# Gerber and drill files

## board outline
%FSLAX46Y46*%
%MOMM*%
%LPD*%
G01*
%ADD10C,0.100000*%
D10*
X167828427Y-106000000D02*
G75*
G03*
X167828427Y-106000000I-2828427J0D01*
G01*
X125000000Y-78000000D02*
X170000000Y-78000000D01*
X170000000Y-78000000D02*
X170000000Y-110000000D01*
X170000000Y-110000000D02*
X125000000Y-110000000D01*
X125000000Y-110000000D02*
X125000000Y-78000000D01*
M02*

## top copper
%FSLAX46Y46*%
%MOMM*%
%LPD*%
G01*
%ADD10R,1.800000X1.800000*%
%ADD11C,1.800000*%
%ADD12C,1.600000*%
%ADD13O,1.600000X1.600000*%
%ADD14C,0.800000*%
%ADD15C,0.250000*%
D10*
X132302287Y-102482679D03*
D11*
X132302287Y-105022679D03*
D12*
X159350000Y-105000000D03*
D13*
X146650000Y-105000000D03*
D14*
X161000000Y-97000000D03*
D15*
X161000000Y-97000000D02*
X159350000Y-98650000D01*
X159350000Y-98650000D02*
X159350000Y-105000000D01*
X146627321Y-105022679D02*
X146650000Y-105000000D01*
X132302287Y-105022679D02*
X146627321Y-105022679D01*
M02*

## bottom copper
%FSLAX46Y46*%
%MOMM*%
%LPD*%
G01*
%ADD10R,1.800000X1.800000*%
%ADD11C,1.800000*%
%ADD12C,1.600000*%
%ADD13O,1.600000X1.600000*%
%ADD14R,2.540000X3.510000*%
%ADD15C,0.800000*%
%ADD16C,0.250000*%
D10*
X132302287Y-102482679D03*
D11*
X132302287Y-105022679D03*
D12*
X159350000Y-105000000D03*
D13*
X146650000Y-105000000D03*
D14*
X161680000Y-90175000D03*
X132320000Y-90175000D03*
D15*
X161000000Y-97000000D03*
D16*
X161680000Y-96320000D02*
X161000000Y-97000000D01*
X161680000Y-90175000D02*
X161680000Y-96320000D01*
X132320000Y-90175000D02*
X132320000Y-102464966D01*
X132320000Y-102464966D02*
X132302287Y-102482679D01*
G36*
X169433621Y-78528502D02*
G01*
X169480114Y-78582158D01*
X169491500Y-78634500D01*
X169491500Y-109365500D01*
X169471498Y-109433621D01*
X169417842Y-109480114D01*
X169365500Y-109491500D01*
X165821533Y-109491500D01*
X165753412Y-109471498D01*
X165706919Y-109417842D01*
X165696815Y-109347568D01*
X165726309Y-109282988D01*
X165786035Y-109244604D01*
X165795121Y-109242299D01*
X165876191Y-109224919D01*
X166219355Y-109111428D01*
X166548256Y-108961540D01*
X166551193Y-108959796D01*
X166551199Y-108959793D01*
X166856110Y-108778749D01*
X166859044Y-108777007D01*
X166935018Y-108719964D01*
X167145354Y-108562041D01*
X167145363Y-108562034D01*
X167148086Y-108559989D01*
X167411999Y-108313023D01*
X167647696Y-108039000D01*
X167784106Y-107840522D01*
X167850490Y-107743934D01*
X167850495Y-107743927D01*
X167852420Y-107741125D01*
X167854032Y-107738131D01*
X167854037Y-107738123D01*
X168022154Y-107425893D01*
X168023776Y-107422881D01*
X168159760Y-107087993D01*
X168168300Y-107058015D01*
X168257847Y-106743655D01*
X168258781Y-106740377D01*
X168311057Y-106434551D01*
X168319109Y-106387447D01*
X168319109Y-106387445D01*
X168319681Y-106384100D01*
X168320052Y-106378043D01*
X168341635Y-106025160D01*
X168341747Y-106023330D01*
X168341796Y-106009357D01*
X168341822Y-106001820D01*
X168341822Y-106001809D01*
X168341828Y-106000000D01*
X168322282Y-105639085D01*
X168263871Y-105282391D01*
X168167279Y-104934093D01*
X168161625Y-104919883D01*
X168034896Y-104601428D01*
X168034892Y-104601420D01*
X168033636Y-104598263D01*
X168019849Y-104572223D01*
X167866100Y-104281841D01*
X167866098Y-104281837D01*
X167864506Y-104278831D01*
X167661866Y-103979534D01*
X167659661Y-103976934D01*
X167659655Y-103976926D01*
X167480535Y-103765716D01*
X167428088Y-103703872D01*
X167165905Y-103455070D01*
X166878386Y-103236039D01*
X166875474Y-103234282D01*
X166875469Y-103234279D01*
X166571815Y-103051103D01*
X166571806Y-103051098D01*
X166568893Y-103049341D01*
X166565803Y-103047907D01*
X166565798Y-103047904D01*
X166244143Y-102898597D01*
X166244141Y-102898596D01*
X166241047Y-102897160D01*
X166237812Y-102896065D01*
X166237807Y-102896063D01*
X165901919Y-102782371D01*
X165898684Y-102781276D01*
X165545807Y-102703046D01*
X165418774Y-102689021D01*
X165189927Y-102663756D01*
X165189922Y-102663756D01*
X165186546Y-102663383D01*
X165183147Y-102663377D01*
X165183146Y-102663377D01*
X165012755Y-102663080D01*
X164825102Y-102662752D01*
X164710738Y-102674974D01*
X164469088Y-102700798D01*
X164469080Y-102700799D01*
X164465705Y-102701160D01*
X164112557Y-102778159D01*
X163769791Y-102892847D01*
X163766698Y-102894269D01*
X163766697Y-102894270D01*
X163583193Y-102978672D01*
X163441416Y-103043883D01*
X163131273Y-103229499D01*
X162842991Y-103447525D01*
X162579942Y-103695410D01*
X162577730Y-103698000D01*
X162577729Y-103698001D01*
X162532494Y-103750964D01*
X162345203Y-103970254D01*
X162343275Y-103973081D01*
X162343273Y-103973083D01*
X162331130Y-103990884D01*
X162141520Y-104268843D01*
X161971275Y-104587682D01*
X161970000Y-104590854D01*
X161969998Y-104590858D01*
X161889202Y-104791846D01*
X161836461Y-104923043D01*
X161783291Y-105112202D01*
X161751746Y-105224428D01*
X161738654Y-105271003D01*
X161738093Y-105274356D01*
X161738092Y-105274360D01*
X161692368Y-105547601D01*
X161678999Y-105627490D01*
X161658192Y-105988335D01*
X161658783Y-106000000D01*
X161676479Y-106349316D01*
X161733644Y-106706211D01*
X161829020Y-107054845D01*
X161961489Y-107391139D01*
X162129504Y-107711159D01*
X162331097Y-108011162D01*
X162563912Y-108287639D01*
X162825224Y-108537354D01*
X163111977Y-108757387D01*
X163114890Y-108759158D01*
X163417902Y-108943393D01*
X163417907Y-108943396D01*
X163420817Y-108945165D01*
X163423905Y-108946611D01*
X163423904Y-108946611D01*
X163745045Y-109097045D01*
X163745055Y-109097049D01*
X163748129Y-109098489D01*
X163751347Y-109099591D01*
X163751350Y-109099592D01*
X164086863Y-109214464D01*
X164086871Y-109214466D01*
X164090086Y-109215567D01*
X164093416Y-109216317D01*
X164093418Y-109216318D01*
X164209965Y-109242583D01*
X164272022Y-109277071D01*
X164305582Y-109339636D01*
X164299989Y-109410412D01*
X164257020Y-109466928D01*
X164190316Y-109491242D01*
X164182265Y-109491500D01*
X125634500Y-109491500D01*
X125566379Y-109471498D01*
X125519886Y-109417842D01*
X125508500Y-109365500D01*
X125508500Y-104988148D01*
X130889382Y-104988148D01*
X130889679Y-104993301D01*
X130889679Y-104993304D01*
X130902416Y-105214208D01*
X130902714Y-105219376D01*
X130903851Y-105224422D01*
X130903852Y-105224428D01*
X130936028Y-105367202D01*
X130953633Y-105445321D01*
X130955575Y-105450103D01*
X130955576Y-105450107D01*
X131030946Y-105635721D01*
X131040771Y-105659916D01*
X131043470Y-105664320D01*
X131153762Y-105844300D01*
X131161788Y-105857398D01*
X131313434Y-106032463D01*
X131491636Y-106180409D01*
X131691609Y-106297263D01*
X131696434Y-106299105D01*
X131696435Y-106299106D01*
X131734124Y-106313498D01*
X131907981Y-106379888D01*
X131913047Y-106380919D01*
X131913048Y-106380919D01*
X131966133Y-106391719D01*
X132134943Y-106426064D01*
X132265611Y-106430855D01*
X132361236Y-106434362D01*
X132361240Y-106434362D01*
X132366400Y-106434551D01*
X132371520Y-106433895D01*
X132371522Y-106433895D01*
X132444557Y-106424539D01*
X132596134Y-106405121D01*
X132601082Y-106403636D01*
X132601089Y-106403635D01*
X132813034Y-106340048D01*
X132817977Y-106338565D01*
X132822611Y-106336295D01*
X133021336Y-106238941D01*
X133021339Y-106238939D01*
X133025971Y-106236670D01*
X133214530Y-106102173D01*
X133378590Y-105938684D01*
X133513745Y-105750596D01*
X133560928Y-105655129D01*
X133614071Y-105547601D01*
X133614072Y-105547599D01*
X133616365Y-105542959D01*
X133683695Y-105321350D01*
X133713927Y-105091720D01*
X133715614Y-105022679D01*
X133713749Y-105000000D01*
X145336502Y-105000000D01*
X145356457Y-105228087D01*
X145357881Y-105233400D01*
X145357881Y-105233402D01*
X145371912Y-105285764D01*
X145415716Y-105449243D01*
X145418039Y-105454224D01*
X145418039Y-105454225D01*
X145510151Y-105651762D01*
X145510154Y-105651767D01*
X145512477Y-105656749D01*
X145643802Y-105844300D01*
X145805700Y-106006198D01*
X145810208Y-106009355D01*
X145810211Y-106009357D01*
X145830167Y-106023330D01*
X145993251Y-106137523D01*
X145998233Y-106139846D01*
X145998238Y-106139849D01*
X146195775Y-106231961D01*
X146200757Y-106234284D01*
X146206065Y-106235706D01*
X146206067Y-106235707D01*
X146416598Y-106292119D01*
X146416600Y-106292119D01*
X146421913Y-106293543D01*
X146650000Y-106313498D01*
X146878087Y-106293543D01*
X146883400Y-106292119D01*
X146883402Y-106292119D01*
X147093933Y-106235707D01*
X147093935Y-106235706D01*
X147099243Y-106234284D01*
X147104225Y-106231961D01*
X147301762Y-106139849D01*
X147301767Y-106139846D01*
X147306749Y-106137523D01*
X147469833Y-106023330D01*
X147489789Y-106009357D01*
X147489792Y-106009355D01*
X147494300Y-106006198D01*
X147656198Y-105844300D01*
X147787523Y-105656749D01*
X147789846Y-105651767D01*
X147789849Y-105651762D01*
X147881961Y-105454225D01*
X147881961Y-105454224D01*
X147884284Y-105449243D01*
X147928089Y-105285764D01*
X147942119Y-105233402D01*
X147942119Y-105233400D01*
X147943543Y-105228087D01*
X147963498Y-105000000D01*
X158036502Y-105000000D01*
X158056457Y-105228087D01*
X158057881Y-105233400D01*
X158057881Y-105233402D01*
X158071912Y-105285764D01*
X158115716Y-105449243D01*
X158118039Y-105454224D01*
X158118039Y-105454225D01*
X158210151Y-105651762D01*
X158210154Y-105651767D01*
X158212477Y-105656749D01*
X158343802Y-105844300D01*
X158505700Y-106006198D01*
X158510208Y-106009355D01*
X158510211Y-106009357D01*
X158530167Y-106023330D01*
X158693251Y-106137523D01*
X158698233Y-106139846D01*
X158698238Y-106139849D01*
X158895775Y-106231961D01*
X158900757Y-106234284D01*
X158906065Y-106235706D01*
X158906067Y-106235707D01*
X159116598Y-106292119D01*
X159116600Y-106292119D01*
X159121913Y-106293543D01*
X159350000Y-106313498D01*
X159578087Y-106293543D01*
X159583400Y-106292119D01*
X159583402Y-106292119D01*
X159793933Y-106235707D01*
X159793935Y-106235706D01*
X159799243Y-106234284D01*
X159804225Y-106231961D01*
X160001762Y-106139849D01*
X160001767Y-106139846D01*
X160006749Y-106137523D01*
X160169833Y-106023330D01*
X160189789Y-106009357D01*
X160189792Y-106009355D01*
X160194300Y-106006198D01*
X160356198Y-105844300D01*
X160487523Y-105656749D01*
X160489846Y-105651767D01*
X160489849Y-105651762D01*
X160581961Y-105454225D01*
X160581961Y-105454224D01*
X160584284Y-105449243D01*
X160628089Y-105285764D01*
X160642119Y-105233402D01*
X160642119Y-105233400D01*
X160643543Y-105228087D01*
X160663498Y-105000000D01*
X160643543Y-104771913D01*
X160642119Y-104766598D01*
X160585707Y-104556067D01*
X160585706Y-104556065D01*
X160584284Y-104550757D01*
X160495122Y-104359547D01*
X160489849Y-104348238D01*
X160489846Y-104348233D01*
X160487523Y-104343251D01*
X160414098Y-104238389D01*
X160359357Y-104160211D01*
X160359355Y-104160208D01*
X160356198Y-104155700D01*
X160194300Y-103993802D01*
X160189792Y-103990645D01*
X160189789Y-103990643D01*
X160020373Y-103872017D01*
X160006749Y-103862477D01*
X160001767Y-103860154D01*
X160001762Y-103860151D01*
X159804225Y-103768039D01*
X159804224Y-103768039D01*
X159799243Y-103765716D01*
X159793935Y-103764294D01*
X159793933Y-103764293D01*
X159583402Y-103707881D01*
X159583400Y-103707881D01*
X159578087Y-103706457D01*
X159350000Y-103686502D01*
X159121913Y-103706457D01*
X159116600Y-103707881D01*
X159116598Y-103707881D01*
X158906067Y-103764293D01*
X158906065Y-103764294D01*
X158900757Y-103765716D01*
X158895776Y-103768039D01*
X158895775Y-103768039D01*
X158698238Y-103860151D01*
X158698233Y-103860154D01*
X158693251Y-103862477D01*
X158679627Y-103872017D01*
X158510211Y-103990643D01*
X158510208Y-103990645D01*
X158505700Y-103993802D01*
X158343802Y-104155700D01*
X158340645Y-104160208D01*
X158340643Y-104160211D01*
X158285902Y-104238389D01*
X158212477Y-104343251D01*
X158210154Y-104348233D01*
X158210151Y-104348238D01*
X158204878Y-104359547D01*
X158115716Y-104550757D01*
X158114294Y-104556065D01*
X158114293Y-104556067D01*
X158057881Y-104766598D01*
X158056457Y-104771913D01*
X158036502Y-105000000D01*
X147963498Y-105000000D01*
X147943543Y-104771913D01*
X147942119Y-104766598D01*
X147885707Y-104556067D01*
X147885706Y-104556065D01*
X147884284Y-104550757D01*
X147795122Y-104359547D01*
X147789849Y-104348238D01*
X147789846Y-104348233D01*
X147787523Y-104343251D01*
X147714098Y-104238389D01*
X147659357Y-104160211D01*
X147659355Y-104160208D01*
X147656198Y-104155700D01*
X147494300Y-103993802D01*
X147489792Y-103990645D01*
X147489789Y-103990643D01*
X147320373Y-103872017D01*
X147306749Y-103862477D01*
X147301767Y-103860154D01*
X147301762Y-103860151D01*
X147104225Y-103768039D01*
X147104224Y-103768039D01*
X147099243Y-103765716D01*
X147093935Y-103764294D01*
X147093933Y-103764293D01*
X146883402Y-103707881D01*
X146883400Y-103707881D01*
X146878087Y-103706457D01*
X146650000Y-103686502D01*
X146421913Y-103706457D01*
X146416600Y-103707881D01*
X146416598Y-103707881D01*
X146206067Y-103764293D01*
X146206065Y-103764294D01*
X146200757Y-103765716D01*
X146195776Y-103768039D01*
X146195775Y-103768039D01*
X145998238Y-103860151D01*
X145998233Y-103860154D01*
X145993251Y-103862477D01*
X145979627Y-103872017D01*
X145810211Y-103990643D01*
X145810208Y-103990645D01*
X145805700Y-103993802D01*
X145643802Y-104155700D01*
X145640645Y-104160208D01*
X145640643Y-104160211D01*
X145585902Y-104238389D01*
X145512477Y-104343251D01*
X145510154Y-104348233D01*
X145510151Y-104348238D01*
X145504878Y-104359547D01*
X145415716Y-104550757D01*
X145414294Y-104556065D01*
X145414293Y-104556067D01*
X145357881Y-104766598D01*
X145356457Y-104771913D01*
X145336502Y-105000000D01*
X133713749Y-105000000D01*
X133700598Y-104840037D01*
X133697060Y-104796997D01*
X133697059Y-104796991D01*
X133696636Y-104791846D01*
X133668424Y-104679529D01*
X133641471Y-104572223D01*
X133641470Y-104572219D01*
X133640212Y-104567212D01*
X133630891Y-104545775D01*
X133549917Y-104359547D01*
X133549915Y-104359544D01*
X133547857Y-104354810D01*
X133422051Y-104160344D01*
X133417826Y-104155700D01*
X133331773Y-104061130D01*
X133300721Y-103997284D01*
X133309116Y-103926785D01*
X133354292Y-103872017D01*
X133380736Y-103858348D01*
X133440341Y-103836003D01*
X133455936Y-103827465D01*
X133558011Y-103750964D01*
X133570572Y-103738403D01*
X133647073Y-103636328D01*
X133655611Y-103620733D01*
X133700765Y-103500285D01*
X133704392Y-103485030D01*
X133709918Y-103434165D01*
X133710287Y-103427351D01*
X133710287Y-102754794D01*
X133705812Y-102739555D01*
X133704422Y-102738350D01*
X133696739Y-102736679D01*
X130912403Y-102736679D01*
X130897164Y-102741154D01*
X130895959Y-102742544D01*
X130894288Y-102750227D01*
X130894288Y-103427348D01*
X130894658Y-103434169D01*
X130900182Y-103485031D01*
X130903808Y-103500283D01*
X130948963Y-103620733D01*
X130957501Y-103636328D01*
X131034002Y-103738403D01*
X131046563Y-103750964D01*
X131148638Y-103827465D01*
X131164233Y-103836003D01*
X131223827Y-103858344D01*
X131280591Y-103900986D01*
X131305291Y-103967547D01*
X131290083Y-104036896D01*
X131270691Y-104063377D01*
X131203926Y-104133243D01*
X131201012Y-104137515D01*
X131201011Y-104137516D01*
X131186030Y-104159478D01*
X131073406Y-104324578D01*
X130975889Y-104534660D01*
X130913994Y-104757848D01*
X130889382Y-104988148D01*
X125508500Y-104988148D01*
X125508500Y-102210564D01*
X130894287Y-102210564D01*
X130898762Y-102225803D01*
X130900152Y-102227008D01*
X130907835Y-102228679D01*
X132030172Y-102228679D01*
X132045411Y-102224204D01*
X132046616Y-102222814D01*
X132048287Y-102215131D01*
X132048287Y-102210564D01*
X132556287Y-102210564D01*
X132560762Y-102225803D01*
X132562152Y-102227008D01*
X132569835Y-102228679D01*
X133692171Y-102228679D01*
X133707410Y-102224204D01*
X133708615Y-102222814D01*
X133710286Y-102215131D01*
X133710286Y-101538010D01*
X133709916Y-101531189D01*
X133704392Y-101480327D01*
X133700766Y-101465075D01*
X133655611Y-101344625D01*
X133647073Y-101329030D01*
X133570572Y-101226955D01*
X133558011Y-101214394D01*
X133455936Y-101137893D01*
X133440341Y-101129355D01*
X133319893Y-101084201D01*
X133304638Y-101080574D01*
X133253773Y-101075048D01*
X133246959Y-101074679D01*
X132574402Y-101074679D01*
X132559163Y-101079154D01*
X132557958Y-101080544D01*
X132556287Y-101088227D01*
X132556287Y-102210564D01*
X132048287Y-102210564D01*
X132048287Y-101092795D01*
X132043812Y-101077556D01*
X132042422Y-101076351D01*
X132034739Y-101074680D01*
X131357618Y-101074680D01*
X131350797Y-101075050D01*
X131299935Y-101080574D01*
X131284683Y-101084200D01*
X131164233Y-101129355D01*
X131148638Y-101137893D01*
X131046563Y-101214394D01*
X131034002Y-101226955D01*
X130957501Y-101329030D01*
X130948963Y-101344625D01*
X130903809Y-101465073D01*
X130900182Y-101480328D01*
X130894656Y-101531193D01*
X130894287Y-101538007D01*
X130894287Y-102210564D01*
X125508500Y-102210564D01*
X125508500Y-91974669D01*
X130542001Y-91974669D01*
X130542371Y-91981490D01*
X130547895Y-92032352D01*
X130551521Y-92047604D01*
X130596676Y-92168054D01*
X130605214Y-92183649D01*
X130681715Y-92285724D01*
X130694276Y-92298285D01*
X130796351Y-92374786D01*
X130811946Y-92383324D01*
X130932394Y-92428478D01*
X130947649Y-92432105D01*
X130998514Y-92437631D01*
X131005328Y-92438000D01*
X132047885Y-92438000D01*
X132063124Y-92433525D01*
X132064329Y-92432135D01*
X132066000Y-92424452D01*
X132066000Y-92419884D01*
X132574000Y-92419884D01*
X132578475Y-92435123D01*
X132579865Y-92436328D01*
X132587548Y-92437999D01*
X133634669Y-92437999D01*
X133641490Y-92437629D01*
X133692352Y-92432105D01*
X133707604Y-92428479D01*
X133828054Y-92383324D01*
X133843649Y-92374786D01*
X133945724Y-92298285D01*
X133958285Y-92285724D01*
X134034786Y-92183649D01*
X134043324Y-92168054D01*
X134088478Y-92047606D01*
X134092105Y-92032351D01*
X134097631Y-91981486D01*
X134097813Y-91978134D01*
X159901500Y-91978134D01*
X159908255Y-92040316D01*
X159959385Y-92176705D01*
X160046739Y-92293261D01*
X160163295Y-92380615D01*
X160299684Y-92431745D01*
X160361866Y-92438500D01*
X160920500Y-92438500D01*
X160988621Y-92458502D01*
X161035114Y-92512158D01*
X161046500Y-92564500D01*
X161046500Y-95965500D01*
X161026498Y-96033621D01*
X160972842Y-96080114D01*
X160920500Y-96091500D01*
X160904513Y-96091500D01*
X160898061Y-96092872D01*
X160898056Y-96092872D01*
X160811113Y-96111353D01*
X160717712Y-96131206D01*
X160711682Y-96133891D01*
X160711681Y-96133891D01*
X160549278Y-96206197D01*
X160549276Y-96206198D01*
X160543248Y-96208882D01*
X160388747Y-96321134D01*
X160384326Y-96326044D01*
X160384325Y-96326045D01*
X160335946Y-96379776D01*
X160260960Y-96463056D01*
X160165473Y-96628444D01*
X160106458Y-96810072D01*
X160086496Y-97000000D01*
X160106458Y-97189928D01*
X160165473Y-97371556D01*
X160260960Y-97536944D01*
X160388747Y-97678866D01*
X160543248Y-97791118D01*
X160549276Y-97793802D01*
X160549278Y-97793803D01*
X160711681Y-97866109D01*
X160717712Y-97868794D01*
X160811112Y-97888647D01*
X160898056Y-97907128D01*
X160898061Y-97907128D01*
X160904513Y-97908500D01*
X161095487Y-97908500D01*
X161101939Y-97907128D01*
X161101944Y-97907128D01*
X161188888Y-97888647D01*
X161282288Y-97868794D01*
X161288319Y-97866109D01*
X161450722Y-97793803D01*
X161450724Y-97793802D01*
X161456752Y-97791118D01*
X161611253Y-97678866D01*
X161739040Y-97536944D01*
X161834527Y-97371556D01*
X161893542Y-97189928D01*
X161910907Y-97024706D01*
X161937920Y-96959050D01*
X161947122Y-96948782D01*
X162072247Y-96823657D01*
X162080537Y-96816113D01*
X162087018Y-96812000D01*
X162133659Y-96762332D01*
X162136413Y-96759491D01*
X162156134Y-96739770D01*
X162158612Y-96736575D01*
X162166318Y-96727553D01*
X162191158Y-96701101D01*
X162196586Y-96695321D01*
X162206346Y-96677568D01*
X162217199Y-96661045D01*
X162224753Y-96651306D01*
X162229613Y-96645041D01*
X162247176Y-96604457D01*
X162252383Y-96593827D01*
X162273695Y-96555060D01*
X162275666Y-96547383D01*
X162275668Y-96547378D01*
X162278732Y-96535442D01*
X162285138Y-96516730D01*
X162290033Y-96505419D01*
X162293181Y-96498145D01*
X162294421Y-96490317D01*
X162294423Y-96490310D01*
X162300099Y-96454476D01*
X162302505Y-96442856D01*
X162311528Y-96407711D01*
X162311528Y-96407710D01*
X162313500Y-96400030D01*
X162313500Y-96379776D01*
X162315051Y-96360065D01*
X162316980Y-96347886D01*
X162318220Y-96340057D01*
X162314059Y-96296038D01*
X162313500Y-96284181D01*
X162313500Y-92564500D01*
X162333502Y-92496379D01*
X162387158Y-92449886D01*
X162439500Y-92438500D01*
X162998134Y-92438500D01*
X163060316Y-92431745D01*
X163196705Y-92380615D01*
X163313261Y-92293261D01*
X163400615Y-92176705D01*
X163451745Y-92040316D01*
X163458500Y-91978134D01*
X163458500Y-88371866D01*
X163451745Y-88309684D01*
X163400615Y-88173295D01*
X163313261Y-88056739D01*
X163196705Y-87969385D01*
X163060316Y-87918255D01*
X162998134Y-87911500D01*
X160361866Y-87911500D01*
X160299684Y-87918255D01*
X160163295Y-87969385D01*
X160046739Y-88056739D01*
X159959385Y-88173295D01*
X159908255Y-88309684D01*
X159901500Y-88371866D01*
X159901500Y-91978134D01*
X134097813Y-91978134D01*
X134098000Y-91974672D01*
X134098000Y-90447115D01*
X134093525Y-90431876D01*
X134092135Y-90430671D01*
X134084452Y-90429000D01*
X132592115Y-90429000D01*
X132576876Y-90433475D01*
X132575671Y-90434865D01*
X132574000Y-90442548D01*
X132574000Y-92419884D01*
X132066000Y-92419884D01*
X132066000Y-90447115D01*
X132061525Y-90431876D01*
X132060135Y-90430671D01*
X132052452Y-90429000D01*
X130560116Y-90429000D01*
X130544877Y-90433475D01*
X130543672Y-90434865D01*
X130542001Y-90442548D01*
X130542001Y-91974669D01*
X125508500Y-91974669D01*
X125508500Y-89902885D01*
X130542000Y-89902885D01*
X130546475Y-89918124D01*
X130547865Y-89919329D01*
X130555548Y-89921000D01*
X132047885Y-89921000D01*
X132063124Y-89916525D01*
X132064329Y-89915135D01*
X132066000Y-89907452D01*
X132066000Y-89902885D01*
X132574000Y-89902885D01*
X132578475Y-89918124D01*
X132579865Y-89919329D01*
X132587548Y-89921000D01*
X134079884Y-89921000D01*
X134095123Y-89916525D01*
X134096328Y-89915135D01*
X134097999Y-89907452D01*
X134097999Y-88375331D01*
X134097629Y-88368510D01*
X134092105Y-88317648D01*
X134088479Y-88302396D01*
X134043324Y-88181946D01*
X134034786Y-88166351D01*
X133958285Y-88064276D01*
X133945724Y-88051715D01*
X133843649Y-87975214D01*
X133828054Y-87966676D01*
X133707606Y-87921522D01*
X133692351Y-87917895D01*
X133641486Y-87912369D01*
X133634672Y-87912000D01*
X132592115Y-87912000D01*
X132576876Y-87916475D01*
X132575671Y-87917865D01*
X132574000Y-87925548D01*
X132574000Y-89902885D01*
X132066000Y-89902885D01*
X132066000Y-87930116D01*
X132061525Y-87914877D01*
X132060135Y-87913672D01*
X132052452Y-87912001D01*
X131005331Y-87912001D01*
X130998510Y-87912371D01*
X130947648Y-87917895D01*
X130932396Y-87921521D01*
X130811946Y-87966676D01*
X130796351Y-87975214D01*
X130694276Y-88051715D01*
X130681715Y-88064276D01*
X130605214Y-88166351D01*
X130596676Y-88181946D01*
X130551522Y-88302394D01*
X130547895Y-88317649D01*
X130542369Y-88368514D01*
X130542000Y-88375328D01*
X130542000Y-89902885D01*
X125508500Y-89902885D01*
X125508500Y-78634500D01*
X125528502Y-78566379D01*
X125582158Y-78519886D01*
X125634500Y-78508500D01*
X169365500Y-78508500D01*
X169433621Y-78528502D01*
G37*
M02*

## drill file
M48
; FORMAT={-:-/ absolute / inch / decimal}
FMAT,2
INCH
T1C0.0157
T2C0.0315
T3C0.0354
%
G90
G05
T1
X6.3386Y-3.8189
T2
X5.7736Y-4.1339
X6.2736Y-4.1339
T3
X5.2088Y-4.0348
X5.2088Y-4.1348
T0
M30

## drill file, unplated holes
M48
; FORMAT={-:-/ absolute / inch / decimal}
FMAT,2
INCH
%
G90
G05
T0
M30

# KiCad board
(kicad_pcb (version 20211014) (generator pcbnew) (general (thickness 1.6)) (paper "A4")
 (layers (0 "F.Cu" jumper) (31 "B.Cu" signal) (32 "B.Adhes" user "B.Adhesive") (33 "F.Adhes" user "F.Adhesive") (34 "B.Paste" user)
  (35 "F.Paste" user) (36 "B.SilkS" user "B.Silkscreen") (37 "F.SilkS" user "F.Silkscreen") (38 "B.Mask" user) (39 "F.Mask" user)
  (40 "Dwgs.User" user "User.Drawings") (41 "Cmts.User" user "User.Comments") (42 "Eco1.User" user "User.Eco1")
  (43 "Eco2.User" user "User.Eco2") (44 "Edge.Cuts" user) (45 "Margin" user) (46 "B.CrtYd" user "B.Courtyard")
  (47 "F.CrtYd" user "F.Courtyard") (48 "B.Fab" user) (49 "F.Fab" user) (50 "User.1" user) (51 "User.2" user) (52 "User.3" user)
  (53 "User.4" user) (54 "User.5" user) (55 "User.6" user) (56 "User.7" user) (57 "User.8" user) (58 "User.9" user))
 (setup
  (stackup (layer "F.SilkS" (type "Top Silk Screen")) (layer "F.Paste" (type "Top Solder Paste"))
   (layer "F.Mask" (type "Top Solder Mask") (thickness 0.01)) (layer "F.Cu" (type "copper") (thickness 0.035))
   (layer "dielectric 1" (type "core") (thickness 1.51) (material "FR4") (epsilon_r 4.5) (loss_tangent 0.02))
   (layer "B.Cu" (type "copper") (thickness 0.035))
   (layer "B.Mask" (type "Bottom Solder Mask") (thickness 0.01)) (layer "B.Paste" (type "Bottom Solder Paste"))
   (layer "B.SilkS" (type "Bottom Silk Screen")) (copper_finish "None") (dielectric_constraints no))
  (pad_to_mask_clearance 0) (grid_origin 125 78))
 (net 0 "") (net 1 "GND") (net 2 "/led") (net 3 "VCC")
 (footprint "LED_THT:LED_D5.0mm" (layer "F.Cu") (at 132.302287 102.482679 -90)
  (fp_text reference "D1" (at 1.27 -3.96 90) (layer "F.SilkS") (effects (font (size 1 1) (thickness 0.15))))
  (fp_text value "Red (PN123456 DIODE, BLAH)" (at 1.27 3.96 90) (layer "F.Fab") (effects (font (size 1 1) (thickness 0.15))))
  (pad "1" thru_hole rect (at 0 0 270) (size 1.8 1.8) (drill 0.9) (layers *.Cu *.Mask) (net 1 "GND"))
  (pad "2" thru_hole circle (at 2.54 0 270) (size 1.8 1.8) (drill 0.9) (layers *.Cu *.Mask) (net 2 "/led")))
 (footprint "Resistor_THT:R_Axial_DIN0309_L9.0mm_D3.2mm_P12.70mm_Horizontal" (layer "F.Cu") (at 159.35 105 180)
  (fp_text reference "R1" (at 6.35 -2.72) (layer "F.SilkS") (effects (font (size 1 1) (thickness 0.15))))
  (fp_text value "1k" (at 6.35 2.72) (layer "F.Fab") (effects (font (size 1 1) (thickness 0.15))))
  (pad "1" thru_hole circle (at 0 0 180) (size 1.6 1.6) (drill 0.8) (layers *.Cu *.Mask) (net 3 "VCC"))
  (pad "2" thru_hole oval (at 12.7 0 180) (size 1.6 1.6) (drill 0.8) (layers *.Cu *.Mask) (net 2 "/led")))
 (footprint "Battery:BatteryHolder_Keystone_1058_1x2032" (layer "B.Cu") (at 147 90.175 180)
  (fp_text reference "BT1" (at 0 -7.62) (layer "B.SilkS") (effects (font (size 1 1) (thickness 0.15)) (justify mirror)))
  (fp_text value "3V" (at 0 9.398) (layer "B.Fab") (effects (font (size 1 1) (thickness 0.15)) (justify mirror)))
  (pad "1" smd rect (at -14.68 0 180) (size 2.54 3.51) (layers "B.Cu" "B.Paste" "B.Mask") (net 3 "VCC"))
  (pad "2" smd rect (at 14.68 0 180) (size 2.54 3.51) (layers "B.Cu" "B.Paste" "B.Mask") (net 1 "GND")))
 (gr_circle (center 165 106) (end 163 108) (layer "Edge.Cuts") (width 0.1) (fill none))
 (gr_rect (start 125 78) (end 170 110) (layer "Edge.Cuts") (width 0.1) (fill none))
 (segment (start 161 97) (end 159.35 98.65) (width 0.25) (layer "F.Cu") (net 3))
 (segment (start 159.35 98.65) (end 159.35 105) (width 0.25) (layer "F.Cu") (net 3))
 (via (at 161 97) (size 0.8) (drill 0.4) (layers "F.Cu" "B.Cu") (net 3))
 (segment (start 161.68 96.32) (end 161 97) (width 0.25) (layer "B.Cu") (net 3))
 (segment (start 161.68 90.175) (end 161.68 96.32) (width 0.25) (layer "B.Cu") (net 3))
 (segment (start 132.32 90.175) (end 132.32 102.464966) (width 0.25) (layer "B.Cu") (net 1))
 (segment (start 132.32 102.464966) (end 132.302287 102.482679) (width 0.25) (layer "B.Cu") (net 1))
 (segment (start 146.627321 105.022679) (end 146.65 105) (width 0.25) (layer "F.Cu") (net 2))
 (segment (start 132.302287 105.022679) (end 146.627321 105.022679) (width 0.25) (layer "F.Cu") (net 2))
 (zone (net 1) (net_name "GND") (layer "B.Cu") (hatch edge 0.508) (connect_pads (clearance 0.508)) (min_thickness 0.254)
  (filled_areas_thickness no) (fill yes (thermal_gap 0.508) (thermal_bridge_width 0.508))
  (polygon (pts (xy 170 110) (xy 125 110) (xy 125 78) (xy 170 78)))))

